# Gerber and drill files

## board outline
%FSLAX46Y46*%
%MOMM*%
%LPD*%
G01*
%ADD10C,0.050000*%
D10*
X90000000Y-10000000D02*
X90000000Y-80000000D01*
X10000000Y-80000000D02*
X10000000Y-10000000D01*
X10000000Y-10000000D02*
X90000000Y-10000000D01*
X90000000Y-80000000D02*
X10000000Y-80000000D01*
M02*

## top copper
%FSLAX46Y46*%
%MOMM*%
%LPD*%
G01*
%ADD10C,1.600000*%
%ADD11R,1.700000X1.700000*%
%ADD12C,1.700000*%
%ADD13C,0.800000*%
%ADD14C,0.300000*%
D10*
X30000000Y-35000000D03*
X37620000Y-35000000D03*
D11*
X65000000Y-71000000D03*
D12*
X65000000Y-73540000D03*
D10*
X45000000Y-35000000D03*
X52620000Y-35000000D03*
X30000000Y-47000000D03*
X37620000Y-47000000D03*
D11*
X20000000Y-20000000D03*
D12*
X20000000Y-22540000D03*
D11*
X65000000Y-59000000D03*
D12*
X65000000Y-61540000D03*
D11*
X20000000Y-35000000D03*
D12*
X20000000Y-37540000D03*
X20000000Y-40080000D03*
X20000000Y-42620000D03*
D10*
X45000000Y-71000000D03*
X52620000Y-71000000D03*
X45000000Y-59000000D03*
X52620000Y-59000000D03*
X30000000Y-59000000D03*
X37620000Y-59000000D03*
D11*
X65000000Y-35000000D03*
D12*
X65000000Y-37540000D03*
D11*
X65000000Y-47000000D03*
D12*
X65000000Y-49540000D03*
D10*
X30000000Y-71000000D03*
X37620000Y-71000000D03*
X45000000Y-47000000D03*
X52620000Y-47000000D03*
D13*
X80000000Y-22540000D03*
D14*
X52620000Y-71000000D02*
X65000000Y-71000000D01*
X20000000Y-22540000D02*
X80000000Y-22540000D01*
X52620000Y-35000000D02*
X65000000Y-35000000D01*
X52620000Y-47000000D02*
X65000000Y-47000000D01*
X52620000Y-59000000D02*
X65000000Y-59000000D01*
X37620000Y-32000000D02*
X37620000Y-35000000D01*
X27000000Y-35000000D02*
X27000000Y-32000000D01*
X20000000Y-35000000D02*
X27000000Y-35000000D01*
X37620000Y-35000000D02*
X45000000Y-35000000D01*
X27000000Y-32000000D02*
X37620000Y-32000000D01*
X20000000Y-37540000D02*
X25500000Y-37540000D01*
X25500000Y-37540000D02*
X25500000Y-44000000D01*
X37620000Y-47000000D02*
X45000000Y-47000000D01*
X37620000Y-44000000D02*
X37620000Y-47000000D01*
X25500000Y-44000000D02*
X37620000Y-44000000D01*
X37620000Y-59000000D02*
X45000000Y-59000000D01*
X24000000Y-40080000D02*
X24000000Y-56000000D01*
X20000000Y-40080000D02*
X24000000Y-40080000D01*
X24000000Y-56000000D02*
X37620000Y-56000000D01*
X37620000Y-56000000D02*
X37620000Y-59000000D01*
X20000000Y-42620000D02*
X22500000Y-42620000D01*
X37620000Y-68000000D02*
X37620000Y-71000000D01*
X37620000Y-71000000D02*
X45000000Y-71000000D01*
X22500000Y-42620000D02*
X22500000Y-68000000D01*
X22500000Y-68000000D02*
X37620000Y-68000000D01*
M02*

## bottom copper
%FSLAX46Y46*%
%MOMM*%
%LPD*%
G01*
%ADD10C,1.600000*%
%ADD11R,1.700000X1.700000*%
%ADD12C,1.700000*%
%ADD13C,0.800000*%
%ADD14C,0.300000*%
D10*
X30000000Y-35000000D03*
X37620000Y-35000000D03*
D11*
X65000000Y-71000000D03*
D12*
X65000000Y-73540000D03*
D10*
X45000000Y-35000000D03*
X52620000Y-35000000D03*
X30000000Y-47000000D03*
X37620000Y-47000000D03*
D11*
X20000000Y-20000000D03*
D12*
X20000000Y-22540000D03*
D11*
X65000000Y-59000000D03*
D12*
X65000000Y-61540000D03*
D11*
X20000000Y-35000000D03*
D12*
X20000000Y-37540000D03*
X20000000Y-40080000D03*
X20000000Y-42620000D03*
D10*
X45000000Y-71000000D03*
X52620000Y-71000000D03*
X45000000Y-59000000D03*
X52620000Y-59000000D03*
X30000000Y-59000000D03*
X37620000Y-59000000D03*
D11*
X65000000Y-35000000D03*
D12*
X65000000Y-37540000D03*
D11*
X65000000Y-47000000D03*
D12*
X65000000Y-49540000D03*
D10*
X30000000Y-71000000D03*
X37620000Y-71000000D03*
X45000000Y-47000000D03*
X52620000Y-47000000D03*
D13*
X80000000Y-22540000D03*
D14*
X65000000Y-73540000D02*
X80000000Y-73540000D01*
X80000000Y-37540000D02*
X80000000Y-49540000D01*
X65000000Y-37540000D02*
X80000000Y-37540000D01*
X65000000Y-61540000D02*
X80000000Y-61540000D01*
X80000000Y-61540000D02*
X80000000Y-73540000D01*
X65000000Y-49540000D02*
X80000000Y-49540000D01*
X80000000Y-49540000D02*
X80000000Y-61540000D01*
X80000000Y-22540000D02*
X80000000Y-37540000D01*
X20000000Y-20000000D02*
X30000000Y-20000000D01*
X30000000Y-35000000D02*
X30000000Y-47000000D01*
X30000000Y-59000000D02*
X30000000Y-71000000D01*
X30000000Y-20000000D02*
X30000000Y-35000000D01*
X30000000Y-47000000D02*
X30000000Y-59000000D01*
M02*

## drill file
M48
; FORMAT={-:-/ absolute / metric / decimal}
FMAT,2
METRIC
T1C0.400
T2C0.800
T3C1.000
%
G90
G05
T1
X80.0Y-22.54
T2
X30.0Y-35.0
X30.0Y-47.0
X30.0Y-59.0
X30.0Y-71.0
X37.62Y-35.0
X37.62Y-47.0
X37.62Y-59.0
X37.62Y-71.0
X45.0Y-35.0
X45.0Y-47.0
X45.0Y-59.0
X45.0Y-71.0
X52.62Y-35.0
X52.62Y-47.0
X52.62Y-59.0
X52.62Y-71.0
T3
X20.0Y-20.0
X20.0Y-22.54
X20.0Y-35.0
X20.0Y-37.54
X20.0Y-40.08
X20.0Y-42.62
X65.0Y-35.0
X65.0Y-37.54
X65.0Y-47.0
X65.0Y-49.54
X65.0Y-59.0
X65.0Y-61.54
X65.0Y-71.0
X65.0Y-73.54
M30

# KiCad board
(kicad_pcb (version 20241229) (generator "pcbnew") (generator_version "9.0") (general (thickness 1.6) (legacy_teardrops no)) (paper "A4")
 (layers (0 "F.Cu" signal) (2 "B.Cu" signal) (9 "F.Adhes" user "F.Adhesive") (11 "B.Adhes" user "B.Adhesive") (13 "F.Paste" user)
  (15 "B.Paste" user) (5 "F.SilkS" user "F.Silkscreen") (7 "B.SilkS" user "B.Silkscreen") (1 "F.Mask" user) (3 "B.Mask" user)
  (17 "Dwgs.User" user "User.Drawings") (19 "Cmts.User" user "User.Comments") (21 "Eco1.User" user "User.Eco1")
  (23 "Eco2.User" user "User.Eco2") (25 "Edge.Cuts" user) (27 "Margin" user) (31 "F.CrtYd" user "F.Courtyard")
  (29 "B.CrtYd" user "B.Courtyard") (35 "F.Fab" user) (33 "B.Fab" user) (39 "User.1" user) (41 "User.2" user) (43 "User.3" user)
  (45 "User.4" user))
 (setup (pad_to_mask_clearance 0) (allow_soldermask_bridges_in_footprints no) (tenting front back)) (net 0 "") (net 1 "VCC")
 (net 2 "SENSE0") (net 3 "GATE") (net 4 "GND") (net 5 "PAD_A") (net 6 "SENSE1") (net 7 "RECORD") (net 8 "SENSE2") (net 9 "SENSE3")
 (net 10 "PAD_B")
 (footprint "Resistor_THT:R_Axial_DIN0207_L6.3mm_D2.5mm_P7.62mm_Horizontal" (layer "F.Cu") (at 30 35)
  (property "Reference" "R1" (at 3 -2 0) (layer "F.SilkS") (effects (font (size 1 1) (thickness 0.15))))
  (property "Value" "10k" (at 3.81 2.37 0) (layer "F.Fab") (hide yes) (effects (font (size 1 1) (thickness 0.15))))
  (pad "1" thru_hole circle (at 0 0) (size 1.6 1.6) (drill 0.8) (layers "*.Cu" "*.Mask") (remove_unused_layers no) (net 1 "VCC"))
  (pad "2" thru_hole circle (at 7.62 0) (size 1.6 1.6) (drill 0.8) (layers "*.Cu" "*.Mask") (remove_unused_layers no) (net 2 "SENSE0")))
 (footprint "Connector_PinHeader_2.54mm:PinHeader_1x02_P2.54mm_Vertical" (layer "F.Cu") (at 65 71)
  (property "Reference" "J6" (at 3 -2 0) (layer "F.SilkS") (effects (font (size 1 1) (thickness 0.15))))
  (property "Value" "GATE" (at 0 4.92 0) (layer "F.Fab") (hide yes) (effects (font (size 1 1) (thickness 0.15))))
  (pad "1" thru_hole rect (at 0 0) (size 1.7 1.7) (drill 1) (layers "*.Cu" "*.Mask") (remove_unused_layers no) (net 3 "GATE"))
  (pad "2" thru_hole circle (at 0 2.54) (size 1.7 1.7) (drill 1) (layers "*.Cu" "*.Mask") (remove_unused_layers no) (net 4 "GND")))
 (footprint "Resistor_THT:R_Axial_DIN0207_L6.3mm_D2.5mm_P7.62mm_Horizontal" (layer "F.Cu") (at 45 35)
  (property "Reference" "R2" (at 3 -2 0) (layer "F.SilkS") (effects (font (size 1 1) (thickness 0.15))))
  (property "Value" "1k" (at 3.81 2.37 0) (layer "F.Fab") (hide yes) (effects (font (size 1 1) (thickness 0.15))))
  (pad "1" thru_hole circle (at 0 0) (size 1.6 1.6) (drill 0.8) (layers "*.Cu" "*.Mask") (remove_unused_layers no) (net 2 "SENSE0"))
  (pad "2" thru_hole circle (at 7.62 0) (size 1.6 1.6) (drill 0.8) (layers "*.Cu" "*.Mask") (remove_unused_layers no) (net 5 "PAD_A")))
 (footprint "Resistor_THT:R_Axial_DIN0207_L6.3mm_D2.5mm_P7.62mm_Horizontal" (layer "F.Cu") (at 30 47)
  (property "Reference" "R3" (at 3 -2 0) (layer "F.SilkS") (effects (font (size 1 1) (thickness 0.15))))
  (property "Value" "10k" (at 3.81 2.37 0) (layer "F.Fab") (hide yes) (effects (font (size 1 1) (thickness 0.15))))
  (pad "1" thru_hole circle (at 0 0) (size 1.6 1.6) (drill 0.8) (layers "*.Cu" "*.Mask") (remove_unused_layers no) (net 1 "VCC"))
  (pad "2" thru_hole circle (at 7.62 0) (size 1.6 1.6) (drill 0.8) (layers "*.Cu" "*.Mask") (remove_unused_layers no) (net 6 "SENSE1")))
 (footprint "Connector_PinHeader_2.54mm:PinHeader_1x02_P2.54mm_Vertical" (layer "F.Cu") (at 20 20)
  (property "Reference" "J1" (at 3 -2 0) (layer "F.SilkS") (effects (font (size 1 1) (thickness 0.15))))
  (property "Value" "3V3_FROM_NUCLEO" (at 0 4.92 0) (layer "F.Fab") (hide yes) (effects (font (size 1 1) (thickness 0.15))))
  (pad "1" thru_hole rect (at 0 0) (size 1.7 1.7) (drill 1) (layers "*.Cu" "*.Mask") (remove_unused_layers no) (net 1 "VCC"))
  (pad "2" thru_hole circle (at 0 2.54) (size 1.7 1.7) (drill 1) (layers "*.Cu" "*.Mask") (remove_unused_layers no) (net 4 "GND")))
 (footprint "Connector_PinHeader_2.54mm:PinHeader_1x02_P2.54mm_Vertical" (layer "F.Cu") (at 65 59)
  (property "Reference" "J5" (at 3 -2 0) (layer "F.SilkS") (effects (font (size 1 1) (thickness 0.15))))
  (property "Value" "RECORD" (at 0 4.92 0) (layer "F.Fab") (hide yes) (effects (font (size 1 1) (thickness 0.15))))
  (pad "1" thru_hole rect (at 0 0) (size 1.7 1.7) (drill 1) (layers "*.Cu" "*.Mask") (remove_unused_layers no) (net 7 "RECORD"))
  (pad "2" thru_hole circle (at 0 2.54) (size 1.7 1.7) (drill 1) (layers "*.Cu" "*.Mask") (remove_unused_layers no) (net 4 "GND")))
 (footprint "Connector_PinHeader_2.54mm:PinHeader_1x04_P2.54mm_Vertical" (layer "F.Cu") (at 20 35)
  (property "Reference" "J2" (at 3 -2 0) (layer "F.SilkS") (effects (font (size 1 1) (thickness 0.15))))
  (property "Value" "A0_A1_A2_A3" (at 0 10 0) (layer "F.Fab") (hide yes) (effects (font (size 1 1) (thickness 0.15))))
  (pad "1" thru_hole rect (at 0 0) (size 1.7 1.7) (drill 1) (layers "*.Cu" "*.Mask") (remove_unused_layers no) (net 2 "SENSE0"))
  (pad "2" thru_hole circle (at 0 2.54) (size 1.7 1.7) (drill 1) (layers "*.Cu" "*.Mask") (remove_unused_layers no) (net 6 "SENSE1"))
  (pad "3" thru_hole circle (at 0 5.08) (size 1.7 1.7) (drill 1) (layers "*.Cu" "*.Mask") (remove_unused_layers no) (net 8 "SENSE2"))
  (pad "4" thru_hole circle (at 0 7.62) (size 1.7 1.7) (drill 1) (layers "*.Cu" "*.Mask") (remove_unused_layers no) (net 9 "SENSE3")))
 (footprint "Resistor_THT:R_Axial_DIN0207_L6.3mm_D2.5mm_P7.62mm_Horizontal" (layer "F.Cu") (at 45 71)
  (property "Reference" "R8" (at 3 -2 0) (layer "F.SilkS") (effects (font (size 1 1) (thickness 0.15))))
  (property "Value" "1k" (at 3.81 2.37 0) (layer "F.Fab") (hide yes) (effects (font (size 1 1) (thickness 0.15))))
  (pad "1" thru_hole circle (at 0 0) (size 1.6 1.6) (drill 0.8) (layers "*.Cu" "*.Mask") (remove_unused_layers no) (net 9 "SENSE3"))
  (pad "2" thru_hole circle (at 7.62 0) (size 1.6 1.6) (drill 0.8) (layers "*.Cu" "*.Mask") (remove_unused_layers no) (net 3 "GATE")))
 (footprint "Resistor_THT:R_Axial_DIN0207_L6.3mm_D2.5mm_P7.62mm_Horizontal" (layer "F.Cu") (at 45 59)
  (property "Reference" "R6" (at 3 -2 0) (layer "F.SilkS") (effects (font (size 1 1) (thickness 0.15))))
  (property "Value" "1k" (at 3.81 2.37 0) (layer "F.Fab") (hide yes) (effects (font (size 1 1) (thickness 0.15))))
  (pad "1" thru_hole circle (at 0 0) (size 1.6 1.6) (drill 0.8) (layers "*.Cu" "*.Mask") (remove_unused_layers no) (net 8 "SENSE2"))
  (pad "2" thru_hole circle (at 7.62 0) (size 1.6 1.6) (drill 0.8) (layers "*.Cu" "*.Mask") (remove_unused_layers no) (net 7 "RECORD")))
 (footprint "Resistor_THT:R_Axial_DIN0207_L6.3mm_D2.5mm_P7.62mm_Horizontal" (layer "F.Cu") (at 30 59)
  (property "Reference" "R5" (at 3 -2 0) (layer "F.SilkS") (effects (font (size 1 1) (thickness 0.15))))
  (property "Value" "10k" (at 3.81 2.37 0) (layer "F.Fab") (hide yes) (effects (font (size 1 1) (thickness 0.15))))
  (pad "1" thru_hole circle (at 0 0) (size 1.6 1.6) (drill 0.8) (layers "*.Cu" "*.Mask") (remove_unused_layers no) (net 1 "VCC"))
  (pad "2" thru_hole circle (at 7.62 0) (size 1.6 1.6) (drill 0.8) (layers "*.Cu" "*.Mask") (remove_unused_layers no) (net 8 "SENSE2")))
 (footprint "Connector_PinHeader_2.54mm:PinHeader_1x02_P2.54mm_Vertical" (layer "F.Cu") (at 65 35)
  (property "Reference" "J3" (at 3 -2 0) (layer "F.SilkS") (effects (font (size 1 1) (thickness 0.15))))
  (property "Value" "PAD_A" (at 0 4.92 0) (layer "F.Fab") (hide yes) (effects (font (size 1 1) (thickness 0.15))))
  (pad "1" thru_hole rect (at 0 0) (size 1.7 1.7) (drill 1) (layers "*.Cu" "*.Mask") (remove_unused_layers no) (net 5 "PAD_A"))
  (pad "2" thru_hole circle (at 0 2.54) (size 1.7 1.7) (drill 1) (layers "*.Cu" "*.Mask") (remove_unused_layers no) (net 4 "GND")))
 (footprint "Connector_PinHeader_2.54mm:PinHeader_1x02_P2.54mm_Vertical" (layer "F.Cu") (at 65 47)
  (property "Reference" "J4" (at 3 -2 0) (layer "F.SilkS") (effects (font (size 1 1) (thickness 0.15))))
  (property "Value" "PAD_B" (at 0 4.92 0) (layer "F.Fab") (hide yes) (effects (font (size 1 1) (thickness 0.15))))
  (pad "1" thru_hole rect (at 0 0) (size 1.7 1.7) (drill 1) (layers "*.Cu" "*.Mask") (remove_unused_layers no) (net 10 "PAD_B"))
  (pad "2" thru_hole circle (at 0 2.54) (size 1.7 1.7) (drill 1) (layers "*.Cu" "*.Mask") (remove_unused_layers no) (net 4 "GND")))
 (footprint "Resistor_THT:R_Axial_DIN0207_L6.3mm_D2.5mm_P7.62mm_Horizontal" (layer "F.Cu") (at 30 71)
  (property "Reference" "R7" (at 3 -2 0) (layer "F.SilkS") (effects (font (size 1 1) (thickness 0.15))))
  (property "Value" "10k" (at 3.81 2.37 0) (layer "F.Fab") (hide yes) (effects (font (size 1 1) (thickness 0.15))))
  (pad "1" thru_hole circle (at 0 0) (size 1.6 1.6) (drill 0.8) (layers "*.Cu" "*.Mask") (remove_unused_layers no) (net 1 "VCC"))
  (pad "2" thru_hole circle (at 7.62 0) (size 1.6 1.6) (drill 0.8) (layers "*.Cu" "*.Mask") (remove_unused_layers no) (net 9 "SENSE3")))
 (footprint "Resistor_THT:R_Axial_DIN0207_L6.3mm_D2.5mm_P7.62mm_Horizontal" (layer "F.Cu") (at 45 47)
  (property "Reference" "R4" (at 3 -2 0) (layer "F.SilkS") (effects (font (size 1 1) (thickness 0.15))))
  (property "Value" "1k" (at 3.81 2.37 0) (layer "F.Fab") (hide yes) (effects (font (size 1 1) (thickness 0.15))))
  (pad "1" thru_hole circle (at 0 0) (size 1.6 1.6) (drill 0.8) (layers "*.Cu" "*.Mask") (remove_unused_layers no) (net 6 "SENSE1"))
  (pad "2" thru_hole circle (at 7.62 0) (size 1.6 1.6) (drill 0.8) (layers "*.Cu" "*.Mask") (remove_unused_layers no) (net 10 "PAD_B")))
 (gr_line (start 90 10) (end 90 80) (stroke (width 0.05) (type default)) (layer "Edge.Cuts"))
 (gr_line (start 10 80) (end 10 10) (stroke (width 0.05) (type default)) (layer "Edge.Cuts"))
 (gr_line (start 10 10) (end 90 10) (stroke (width 0.05) (type default)) (layer "Edge.Cuts"))
 (gr_line (start 90 80) (end 10 80) (stroke (width 0.05) (type default)) (layer "Edge.Cuts"))
 (segment (start 52.62 71) (end 65 71) (width 0.3) (layer "F.Cu") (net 3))
 (segment (start 20 22.54) (end 80 22.54) (width 0.3) (layer "F.Cu") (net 4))
 (via (at 80 22.54) (size 0.8) (drill 0.4) (layers "F.Cu" "B.Cu") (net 4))
 (segment (start 65 73.54) (end 80 73.54) (width 0.3) (layer "B.Cu") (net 4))
 (segment (start 80 37.54) (end 80 49.54) (width 0.3) (layer "B.Cu") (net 4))
 (segment (start 65 37.54) (end 80 37.54) (width 0.3) (layer "B.Cu") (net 4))
 (segment (start 65 61.54) (end 80 61.54) (width 0.3) (layer "B.Cu") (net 4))
 (segment (start 80 61.54) (end 80 73.54) (width 0.3) (layer "B.Cu") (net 4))
 (segment (start 65 49.54) (end 80 49.54) (width 0.3) (layer "B.Cu") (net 4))
 (segment (start 80 49.54) (end 80 61.54) (width 0.3) (layer "B.Cu") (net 4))
 (segment (start 80 22.54) (end 80 37.54) (width 0.3) (layer "B.Cu") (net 4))
 (segment (start 52.62 35) (end 65 35) (width 0.3) (layer "F.Cu") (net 5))
 (segment (start 52.62 47) (end 65 47) (width 0.3) (layer "F.Cu") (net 10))
 (segment (start 52.62 59) (end 65 59) (width 0.3) (layer "F.Cu") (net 7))
 (segment (start 37.62 32) (end 37.62 35) (width 0.3) (layer "F.Cu") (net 2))
 (segment (start 27 35) (end 27 32) (width 0.3) (layer "F.Cu") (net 2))
 (segment (start 20 35) (end 27 35) (width 0.3) (layer "F.Cu") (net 2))
 (segment (start 37.62 35) (end 45 35) (width 0.3) (layer "F.Cu") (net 2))
 (segment (start 27 32) (end 37.62 32) (width 0.3) (layer "F.Cu") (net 2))
 (segment (start 20 37.54) (end 25.5 37.54) (width 0.3) (layer "F.Cu") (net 6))
 (segment (start 25.5 37.54) (end 25.5 44) (width 0.3) (layer "F.Cu") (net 6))
 (segment (start 37.62 47) (end 45 47) (width 0.3) (layer "F.Cu") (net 6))
 (segment (start 37.62 44) (end 37.62 47) (width 0.3) (layer "F.Cu") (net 6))
 (segment (start 25.5 44) (end 37.62 44) (width 0.3) (layer "F.Cu") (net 6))
 (segment (start 37.62 59) (end 45 59) (width 0.3) (layer "F.Cu") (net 8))
 (segment (start 24 40.08) (end 24 56) (width 0.3) (layer "F.Cu") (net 8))
 (segment (start 20 40.08) (end 24 40.08) (width 0.3) (layer "F.Cu") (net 8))
 (segment (start 24 56) (end 37.62 56) (width 0.3) (layer "F.Cu") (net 8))
 (segment (start 37.62 56) (end 37.62 59) (width 0.3) (layer "F.Cu") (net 8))
 (segment (start 20 42.62) (end 22.5 42.62) (width 0.3) (layer "F.Cu") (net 9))
 (segment (start 37.62 68) (end 37.62 71) (width 0.3) (layer "F.Cu") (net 9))
 (segment (start 37.62 71) (end 45 71) (width 0.3) (layer "F.Cu") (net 9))
 (segment (start 22.5 42.62) (end 22.5 68) (width 0.3) (layer "F.Cu") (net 9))
 (segment (start 22.5 68) (end 37.62 68) (width 0.3) (layer "F.Cu") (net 9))
 (segment (start 20 20) (end 30 20) (width 0.3) (layer "B.Cu") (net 1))
 (segment (start 30 35) (end 30 47) (width 0.3) (layer "B.Cu") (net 1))
 (segment (start 30 59) (end 30 71) (width 0.3) (layer "B.Cu") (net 1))
 (segment (start 30 20) (end 30 35) (width 0.3) (layer "B.Cu") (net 1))
 (segment (start 30 47) (end 30 59) (width 0.3) (layer "B.Cu") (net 1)))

